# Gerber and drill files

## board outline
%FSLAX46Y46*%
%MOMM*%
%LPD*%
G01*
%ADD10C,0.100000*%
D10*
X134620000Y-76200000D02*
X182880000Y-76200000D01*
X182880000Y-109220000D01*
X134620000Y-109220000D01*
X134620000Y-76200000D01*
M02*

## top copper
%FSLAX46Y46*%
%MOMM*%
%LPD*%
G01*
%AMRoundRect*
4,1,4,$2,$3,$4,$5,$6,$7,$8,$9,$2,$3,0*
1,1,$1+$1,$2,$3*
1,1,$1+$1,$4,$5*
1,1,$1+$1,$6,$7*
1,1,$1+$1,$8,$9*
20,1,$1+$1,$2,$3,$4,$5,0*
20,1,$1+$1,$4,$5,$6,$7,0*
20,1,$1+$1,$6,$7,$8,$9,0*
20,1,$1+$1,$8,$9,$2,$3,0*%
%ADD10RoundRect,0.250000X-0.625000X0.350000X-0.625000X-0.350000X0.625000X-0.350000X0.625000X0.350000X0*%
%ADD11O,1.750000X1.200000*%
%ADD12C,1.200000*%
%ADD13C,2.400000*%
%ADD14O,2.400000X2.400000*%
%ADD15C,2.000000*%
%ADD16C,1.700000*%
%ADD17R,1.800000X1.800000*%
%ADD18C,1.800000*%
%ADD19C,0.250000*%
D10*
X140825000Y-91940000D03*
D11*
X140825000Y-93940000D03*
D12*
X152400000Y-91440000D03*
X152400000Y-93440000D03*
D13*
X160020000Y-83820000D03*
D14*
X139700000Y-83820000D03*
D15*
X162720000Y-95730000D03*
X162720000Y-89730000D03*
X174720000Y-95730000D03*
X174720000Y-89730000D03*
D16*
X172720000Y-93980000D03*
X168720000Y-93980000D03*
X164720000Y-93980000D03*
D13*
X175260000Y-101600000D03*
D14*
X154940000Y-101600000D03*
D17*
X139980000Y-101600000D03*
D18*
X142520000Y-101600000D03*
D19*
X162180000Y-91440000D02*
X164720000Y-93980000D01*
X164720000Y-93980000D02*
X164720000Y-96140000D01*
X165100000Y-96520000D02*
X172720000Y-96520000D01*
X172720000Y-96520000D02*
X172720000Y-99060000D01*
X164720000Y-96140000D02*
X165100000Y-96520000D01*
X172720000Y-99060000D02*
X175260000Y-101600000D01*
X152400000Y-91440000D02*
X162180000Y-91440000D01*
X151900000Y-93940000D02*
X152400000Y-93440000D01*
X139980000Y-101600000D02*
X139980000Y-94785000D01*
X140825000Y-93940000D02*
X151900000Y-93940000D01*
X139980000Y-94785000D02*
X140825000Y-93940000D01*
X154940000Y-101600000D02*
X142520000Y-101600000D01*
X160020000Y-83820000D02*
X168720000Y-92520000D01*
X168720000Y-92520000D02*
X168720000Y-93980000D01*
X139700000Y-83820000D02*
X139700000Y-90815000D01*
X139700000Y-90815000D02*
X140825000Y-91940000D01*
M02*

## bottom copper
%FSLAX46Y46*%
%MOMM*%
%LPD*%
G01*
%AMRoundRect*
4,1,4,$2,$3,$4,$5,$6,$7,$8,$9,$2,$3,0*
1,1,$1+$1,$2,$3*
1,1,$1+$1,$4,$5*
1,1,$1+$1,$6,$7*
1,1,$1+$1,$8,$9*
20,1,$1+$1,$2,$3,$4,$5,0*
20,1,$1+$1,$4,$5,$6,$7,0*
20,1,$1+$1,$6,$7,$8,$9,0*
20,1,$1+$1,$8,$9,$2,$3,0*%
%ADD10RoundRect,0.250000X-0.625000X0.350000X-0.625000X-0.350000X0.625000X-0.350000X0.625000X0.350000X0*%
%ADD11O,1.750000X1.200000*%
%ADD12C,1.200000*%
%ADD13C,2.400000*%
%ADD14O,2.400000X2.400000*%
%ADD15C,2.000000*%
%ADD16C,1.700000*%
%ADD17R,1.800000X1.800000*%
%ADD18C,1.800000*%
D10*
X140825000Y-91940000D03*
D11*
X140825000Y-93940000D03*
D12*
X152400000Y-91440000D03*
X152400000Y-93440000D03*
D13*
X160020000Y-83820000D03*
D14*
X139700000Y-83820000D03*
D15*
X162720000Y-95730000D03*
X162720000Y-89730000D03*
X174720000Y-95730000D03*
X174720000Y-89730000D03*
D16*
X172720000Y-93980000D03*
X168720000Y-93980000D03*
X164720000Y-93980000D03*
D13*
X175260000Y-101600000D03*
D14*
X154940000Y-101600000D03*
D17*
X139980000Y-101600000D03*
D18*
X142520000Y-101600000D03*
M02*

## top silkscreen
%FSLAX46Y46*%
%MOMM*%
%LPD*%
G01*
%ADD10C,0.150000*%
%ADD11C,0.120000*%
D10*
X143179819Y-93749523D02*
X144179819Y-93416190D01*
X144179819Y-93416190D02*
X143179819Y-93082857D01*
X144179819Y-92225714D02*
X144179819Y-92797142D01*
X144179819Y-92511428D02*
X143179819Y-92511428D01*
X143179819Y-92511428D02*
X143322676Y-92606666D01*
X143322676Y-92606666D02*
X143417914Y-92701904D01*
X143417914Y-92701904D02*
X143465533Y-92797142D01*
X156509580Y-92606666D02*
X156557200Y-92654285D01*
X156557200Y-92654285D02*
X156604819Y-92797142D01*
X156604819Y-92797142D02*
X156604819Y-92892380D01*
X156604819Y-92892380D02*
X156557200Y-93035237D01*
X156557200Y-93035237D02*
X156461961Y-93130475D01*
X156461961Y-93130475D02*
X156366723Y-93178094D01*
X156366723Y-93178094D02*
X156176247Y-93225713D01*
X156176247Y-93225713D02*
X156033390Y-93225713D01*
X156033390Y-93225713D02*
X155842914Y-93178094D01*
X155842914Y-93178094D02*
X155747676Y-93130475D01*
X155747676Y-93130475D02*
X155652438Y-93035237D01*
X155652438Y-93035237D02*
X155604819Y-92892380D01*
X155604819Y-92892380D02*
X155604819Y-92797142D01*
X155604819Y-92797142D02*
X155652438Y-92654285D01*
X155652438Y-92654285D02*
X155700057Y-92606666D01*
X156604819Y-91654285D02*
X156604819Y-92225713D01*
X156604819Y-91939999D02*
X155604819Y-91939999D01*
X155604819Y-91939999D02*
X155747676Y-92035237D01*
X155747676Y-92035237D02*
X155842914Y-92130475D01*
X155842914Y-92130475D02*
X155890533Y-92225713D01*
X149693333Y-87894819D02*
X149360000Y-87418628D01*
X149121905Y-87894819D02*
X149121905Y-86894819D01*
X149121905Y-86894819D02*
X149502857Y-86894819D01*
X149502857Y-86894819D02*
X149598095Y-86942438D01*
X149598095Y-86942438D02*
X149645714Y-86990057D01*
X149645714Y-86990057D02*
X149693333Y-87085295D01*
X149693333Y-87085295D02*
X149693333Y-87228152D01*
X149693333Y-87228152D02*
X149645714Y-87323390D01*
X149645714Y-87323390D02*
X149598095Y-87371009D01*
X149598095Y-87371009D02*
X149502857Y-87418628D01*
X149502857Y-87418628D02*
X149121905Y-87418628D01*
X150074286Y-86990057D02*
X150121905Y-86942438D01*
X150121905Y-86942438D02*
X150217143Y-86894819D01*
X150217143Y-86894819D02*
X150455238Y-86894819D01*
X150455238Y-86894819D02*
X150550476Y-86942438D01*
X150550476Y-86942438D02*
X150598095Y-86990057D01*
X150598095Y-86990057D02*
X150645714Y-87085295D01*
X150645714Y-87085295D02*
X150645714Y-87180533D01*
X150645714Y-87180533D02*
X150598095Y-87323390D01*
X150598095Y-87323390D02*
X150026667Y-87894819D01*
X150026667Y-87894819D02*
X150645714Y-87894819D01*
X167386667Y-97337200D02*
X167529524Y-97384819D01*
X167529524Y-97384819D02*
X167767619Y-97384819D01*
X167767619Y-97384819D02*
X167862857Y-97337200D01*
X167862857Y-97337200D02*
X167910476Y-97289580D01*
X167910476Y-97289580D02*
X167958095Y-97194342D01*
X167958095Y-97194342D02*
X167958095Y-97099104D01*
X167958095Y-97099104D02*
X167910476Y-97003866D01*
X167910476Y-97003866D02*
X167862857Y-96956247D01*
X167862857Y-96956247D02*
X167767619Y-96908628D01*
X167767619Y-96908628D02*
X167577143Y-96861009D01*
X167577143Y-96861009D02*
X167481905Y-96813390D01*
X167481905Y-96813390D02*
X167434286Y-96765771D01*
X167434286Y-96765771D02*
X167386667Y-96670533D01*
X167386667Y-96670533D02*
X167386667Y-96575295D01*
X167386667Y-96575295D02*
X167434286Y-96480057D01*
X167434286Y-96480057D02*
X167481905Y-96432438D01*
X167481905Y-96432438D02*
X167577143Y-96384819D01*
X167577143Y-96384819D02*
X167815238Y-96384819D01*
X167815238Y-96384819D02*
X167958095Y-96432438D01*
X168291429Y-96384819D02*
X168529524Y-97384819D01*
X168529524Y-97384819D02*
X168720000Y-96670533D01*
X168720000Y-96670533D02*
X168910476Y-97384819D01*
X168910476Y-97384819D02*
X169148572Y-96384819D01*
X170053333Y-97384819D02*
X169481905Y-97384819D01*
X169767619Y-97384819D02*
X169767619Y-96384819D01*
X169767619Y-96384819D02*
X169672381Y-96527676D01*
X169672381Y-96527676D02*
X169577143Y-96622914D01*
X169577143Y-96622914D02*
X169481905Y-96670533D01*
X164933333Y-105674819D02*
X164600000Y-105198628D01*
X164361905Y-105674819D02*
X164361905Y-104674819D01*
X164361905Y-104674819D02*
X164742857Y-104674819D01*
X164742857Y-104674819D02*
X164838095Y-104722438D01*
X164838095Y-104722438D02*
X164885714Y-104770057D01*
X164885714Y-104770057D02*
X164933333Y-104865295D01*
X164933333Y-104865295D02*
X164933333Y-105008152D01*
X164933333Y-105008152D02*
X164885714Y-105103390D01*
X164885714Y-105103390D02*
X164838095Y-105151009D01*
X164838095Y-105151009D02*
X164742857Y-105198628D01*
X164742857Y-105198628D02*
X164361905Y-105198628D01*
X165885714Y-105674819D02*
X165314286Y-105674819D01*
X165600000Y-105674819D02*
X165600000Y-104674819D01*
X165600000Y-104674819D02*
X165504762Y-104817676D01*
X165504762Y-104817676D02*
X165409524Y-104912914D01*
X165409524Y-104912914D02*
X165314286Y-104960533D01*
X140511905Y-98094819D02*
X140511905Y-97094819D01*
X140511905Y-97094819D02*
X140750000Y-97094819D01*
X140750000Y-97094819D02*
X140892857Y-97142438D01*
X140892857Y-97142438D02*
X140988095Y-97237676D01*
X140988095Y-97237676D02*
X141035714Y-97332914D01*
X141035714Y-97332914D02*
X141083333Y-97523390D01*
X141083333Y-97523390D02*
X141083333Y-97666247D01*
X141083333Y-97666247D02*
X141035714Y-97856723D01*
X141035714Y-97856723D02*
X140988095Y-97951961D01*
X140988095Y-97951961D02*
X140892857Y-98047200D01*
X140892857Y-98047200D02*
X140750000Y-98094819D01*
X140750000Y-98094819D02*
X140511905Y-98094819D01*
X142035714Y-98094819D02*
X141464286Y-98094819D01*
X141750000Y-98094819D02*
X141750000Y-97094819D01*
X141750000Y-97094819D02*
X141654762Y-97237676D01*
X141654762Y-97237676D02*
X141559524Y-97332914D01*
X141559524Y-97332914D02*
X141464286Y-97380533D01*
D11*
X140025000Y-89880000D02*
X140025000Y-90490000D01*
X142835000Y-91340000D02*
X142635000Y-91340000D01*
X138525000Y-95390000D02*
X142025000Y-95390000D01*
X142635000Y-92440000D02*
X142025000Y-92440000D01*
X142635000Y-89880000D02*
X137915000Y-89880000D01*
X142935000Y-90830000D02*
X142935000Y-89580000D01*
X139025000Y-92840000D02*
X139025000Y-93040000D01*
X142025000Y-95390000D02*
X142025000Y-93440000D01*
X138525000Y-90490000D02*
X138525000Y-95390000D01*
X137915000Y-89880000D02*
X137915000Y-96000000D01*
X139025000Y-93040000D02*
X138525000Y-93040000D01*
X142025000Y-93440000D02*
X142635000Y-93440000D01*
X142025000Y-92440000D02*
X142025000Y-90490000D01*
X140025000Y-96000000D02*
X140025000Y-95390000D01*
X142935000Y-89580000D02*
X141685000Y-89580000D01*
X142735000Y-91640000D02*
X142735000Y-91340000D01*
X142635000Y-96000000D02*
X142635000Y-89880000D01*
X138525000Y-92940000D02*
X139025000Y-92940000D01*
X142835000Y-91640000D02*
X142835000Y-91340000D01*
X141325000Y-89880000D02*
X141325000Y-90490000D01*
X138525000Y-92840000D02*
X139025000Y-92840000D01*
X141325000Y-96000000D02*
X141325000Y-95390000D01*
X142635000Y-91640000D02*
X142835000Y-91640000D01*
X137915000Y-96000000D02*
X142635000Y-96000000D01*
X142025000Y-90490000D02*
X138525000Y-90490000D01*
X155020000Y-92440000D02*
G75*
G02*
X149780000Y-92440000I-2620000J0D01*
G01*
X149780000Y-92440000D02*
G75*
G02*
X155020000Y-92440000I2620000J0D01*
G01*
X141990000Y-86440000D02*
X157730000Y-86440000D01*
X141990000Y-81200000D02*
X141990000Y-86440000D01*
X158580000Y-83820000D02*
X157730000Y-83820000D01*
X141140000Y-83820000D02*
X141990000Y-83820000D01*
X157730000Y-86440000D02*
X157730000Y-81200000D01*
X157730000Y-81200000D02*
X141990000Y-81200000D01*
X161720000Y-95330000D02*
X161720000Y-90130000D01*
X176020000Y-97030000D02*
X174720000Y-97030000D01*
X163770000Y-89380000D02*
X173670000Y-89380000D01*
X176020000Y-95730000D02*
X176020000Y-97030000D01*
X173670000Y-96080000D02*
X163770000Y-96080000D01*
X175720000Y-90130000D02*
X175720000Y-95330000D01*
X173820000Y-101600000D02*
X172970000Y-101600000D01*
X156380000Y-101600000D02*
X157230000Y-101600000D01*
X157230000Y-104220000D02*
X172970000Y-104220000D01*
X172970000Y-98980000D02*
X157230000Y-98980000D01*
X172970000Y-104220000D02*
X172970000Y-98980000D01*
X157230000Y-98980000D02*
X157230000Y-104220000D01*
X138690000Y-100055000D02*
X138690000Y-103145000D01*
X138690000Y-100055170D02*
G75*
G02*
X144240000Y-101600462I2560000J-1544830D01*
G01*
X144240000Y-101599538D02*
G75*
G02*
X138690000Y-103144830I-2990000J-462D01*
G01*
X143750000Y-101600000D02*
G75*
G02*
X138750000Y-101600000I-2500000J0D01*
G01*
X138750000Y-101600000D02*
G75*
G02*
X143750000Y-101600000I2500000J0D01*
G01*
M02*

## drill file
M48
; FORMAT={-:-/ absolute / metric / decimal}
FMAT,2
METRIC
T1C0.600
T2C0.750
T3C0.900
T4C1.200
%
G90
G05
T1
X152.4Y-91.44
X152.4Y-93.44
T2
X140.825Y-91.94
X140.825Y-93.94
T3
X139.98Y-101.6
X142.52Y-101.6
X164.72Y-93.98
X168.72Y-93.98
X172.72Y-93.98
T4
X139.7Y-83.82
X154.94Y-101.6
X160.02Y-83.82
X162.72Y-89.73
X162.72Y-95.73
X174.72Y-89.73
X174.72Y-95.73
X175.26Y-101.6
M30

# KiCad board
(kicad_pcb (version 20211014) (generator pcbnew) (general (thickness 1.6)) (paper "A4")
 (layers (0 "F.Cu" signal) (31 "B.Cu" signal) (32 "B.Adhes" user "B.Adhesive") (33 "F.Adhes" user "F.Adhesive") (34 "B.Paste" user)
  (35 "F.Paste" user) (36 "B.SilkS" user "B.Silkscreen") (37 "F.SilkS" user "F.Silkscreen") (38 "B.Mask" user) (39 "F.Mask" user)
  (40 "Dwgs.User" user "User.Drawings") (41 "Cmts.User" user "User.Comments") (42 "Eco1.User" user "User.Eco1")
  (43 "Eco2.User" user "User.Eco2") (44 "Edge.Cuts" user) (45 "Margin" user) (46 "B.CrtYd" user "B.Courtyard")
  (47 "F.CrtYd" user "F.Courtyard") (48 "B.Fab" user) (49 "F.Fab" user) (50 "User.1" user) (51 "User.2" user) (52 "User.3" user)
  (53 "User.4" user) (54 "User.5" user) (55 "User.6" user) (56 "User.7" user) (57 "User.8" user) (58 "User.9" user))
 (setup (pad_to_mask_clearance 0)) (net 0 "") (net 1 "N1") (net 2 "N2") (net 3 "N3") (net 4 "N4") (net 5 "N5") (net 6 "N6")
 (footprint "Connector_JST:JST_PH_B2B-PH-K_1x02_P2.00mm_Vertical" (layer "F.Cu") (at 140.825 91.94 -90)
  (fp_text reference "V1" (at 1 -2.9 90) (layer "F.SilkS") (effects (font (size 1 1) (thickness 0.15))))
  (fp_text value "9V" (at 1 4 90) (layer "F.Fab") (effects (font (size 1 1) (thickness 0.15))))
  (fp_line (start -2.06 0.8) (end -1.45 0.8) (layer "F.SilkS") (width 0.12))
  (fp_line (start -0.6 -2.01) (end -0.6 -1.81) (layer "F.SilkS") (width 0.12))
  (fp_line (start 3.45 2.3) (end 3.45 -1.2) (layer "F.SilkS") (width 0.12))
  (fp_line (start 0.5 -1.81) (end 0.5 -1.2) (layer "F.SilkS") (width 0.12))
  (fp_line (start -2.06 -1.81) (end -2.06 2.91) (layer "F.SilkS") (width 0.12))
  (fp_line (start -1.11 -2.11) (end -2.36 -2.11) (layer "F.SilkS") (width 0.12))
  (fp_line (start 0.9 1.8) (end 1.1 1.8) (layer "F.SilkS") (width 0.12))
  (fp_line (start 3.45 -1.2) (end 1.5 -1.2) (layer "F.SilkS") (width 0.12))
  (fp_line (start -1.45 2.3) (end 3.45 2.3) (layer "F.SilkS") (width 0.12))
  (fp_line (start -2.06 2.91) (end 4.06 2.91) (layer "F.SilkS") (width 0.12))
  (fp_line (start 1.1 1.8) (end 1.1 2.3) (layer "F.SilkS") (width 0.12))
  (fp_line (start 1.5 -1.2) (end 1.5 -1.81) (layer "F.SilkS") (width 0.12))
  (fp_line (start 0.5 -1.2) (end -1.45 -1.2) (layer "F.SilkS") (width 0.12))
  (fp_line (start 4.06 0.8) (end 3.45 0.8) (layer "F.SilkS") (width 0.12))
  (fp_line (start -2.36 -2.11) (end -2.36 -0.86) (layer "F.SilkS") (width 0.12))
  (fp_line (start -0.3 -1.91) (end -0.6 -1.91) (layer "F.SilkS") (width 0.12))
  (fp_line (start 4.06 -1.81) (end -2.06 -1.81) (layer "F.SilkS") (width 0.12))
  (fp_line (start 1 2.3) (end 1 1.8) (layer "F.SilkS") (width 0.12))
  (fp_line (start -0.3 -2.01) (end -0.6 -2.01) (layer "F.SilkS") (width 0.12))
  (fp_line (start -2.06 -0.5) (end -1.45 -0.5) (layer "F.SilkS") (width 0.12))
  (fp_line (start 0.9 2.3) (end 0.9 1.8) (layer "F.SilkS") (width 0.12))
  (fp_line (start 4.06 -0.5) (end 3.45 -0.5) (layer "F.SilkS") (width 0.12))
  (fp_line (start -0.3 -1.81) (end -0.3 -2.01) (layer "F.SilkS") (width 0.12))
  (fp_line (start 4.06 2.91) (end 4.06 -1.81) (layer "F.SilkS") (width 0.12))
  (fp_line (start -1.45 -1.2) (end -1.45 2.3) (layer "F.SilkS") (width 0.12))
  (pad "1" thru_hole roundrect (at 0 0 270) (size 1.2 1.75) (drill 0.75) (layers *.Cu *.Mask) (roundrect_rratio 0.208333) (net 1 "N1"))
  (pad "2" thru_hole oval (at 2 0 270) (size 1.2 1.75) (drill 0.75) (layers *.Cu *.Mask) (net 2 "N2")))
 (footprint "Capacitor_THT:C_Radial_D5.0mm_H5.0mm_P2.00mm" (layer "F.Cu") (at 152.4 91.44 -90)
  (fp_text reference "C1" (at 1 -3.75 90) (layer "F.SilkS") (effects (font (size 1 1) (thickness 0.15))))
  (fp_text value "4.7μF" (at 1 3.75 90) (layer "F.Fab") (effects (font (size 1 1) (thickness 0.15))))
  (fp_circle (center 1 0) (end 3.62 0) (layer "F.SilkS") (width 0.12) (fill none))
  (pad "1" thru_hole circle (at 0 0 270) (size 1.2 1.2) (drill 0.6) (layers *.Cu *.Mask) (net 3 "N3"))
  (pad "2" thru_hole circle (at 2 0 270) (size 1.2 1.2) (drill 0.6) (layers *.Cu *.Mask) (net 2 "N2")))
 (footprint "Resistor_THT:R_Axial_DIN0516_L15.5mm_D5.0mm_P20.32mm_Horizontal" (layer "F.Cu") (at 160.02 83.82 180)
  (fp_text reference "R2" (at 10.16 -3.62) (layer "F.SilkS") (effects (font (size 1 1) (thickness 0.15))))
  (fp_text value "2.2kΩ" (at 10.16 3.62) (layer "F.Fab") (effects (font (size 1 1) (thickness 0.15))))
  (fp_line (start 18.03 -2.62) (end 2.29 -2.62) (layer "F.SilkS") (width 0.12))
  (fp_line (start 18.03 2.62) (end 18.03 -2.62) (layer "F.SilkS") (width 0.12))
  (fp_line (start 1.44 0) (end 2.29 0) (layer "F.SilkS") (width 0.12))
  (fp_line (start 18.88 0) (end 18.03 0) (layer "F.SilkS") (width 0.12))
  (fp_line (start 2.29 -2.62) (end 2.29 2.62) (layer "F.SilkS") (width 0.12))
  (fp_line (start 2.29 2.62) (end 18.03 2.62) (layer "F.SilkS") (width 0.12))
  (pad "1" thru_hole circle (at 0 0 180) (size 2.4 2.4) (drill 1.2) (layers *.Cu *.Mask) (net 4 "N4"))
  (pad "2" thru_hole oval (at 20.32 0 180) (size 2.4 2.4) (drill 1.2) (layers *.Cu *.Mask) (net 1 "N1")))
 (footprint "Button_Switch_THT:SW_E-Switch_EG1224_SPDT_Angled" (layer "F.Cu") (at 172.72 93.98 180)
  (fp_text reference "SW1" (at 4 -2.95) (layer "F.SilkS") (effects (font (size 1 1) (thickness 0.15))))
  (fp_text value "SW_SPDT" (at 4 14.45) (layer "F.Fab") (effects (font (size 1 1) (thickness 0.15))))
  (fp_line (start 11 -1.35) (end 11 3.85) (layer "F.SilkS") (width 0.12))
  (fp_line (start -3.3 -3.05) (end -2 -3.05) (layer "F.SilkS") (width 0.12))
  (fp_line (start 8.95 4.6) (end -0.95 4.6) (layer "F.SilkS") (width 0.12))
  (fp_line (start -3.3 -1.75) (end -3.3 -3.05) (layer "F.SilkS") (width 0.12))
  (fp_line (start -0.95 -2.1) (end 8.95 -2.1) (layer "F.SilkS") (width 0.12))
  (fp_line (start -3 3.85) (end -3 -1.35) (layer "F.SilkS") (width 0.12))
  (pad "" thru_hole circle (at 10 -1.75 180) (size 2 2) (drill 1.2) (layers *.Cu *.Mask))
  (pad "" thru_hole circle (at 10 4.25 180) (size 2 2) (drill 1.2) (layers *.Cu *.Mask))
  (pad "" thru_hole circle (at -2 -1.75 180) (size 2 2) (drill 1.2) (layers *.Cu *.Mask))
  (pad "" thru_hole circle (at -2 4.25 180) (size 2 2) (drill 1.2) (layers *.Cu *.Mask))
  (pad "1" thru_hole circle (at 0 0 180) (size 1.7 1.7) (drill 0.9) (layers *.Cu *.Mask) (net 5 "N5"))
  (pad "2" thru_hole circle (at 4 0 180) (size 1.7 1.7) (drill 0.9) (layers *.Cu *.Mask) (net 4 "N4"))
  (pad "3" thru_hole circle (at 8 0 180) (size 1.7 1.7) (drill 0.9) (layers *.Cu *.Mask) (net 3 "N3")))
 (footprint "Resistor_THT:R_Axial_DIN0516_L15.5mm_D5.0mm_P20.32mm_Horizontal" (layer "F.Cu") (at 175.26 101.6 180)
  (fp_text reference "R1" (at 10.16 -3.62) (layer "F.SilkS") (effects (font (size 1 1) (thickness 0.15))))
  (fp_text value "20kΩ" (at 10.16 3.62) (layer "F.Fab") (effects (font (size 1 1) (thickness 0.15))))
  (fp_line (start 1.44 0) (end 2.29 0) (layer "F.SilkS") (width 0.12))
  (fp_line (start 18.88 0) (end 18.03 0) (layer "F.SilkS") (width 0.12))
  (fp_line (start 18.03 -2.62) (end 2.29 -2.62) (layer "F.SilkS") (width 0.12))
  (fp_line (start 2.29 2.62) (end 18.03 2.62) (layer "F.SilkS") (width 0.12))
  (fp_line (start 2.29 -2.62) (end 2.29 2.62) (layer "F.SilkS") (width 0.12))
  (fp_line (start 18.03 2.62) (end 18.03 -2.62) (layer "F.SilkS") (width 0.12))
  (pad "1" thru_hole circle (at 0 0 180) (size 2.4 2.4) (drill 1.2) (layers *.Cu *.Mask) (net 3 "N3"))
  (pad "2" thru_hole oval (at 20.32 0 180) (size 2.4 2.4) (drill 1.2) (layers *.Cu *.Mask) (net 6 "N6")))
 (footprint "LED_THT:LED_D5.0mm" (layer "F.Cu") (at 139.98 101.6)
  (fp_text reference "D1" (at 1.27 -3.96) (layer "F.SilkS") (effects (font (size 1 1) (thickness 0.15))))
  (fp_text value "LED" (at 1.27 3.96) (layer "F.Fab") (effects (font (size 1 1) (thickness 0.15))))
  (fp_line (start -1.29 -1.545) (end -1.29 1.545) (layer "F.SilkS") (width 0.12))
  (fp_arc (start -1.29 -1.54483) (mid 2.072002 -2.880433) (end 4.26 0.000462) (layer "F.SilkS") (width 0.12))
  (fp_arc (start 4.26 -0.000462) (mid 2.072002 2.880433) (end -1.29 1.54483) (layer "F.SilkS") (width 0.12))
  (fp_circle (center 1.27 0) (end 3.77 0) (layer "F.SilkS") (width 0.12) (fill none))
  (pad "1" thru_hole rect (at 0 0) (size 1.8 1.8) (drill 0.9) (layers *.Cu *.Mask) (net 2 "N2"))
  (pad "2" thru_hole circle (at 2.54 0) (size 1.8 1.8) (drill 0.9) (layers *.Cu *.Mask) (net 6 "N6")))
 (gr_rect (start 134.62 76.2) (end 182.88 109.22) (layer "Edge.Cuts") (width 0.1) (fill none))
 (segment (start 162.18 91.44) (end 164.72 93.98) (width 0.25) (layer "F.Cu") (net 3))
 (segment (start 164.72 93.98) (end 164.72 96.14) (width 0.25) (layer "F.Cu") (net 3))
 (segment (start 165.1 96.52) (end 172.72 96.52) (width 0.25) (layer "F.Cu") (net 3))
 (segment (start 172.72 96.52) (end 172.72 99.06) (width 0.25) (layer "F.Cu") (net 3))
 (segment (start 164.72 96.14) (end 165.1 96.52) (width 0.25) (layer "F.Cu") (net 3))
 (segment (start 172.72 99.06) (end 175.26 101.6) (width 0.25) (layer "F.Cu") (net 3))
 (segment (start 152.4 91.44) (end 162.18 91.44) (width 0.25) (layer "F.Cu") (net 3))
 (segment (start 151.9 93.94) (end 152.4 93.44) (width 0.25) (layer "F.Cu") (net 2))
 (segment (start 139.98 101.6) (end 139.98 94.785) (width 0.25) (layer "F.Cu") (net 2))
 (segment (start 140.825 93.94) (end 151.9 93.94) (width 0.25) (layer "F.Cu") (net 2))
 (segment (start 139.98 94.785) (end 140.825 93.94) (width 0.25) (layer "F.Cu") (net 2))
 (segment (start 154.94 101.6) (end 142.52 101.6) (width 0.25) (layer "F.Cu") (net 6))
 (segment (start 160.02 83.82) (end 168.72 92.52) (width 0.25) (layer "F.Cu") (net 4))
 (segment (start 168.72 92.52) (end 168.72 93.98) (width 0.25) (layer "F.Cu") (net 4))
 (segment (start 139.7 83.82) (end 139.7 90.815) (width 0.25) (layer "F.Cu") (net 1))
 (segment (start 139.7 90.815) (end 140.825 91.94) (width 0.25) (layer "F.Cu") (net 1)))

